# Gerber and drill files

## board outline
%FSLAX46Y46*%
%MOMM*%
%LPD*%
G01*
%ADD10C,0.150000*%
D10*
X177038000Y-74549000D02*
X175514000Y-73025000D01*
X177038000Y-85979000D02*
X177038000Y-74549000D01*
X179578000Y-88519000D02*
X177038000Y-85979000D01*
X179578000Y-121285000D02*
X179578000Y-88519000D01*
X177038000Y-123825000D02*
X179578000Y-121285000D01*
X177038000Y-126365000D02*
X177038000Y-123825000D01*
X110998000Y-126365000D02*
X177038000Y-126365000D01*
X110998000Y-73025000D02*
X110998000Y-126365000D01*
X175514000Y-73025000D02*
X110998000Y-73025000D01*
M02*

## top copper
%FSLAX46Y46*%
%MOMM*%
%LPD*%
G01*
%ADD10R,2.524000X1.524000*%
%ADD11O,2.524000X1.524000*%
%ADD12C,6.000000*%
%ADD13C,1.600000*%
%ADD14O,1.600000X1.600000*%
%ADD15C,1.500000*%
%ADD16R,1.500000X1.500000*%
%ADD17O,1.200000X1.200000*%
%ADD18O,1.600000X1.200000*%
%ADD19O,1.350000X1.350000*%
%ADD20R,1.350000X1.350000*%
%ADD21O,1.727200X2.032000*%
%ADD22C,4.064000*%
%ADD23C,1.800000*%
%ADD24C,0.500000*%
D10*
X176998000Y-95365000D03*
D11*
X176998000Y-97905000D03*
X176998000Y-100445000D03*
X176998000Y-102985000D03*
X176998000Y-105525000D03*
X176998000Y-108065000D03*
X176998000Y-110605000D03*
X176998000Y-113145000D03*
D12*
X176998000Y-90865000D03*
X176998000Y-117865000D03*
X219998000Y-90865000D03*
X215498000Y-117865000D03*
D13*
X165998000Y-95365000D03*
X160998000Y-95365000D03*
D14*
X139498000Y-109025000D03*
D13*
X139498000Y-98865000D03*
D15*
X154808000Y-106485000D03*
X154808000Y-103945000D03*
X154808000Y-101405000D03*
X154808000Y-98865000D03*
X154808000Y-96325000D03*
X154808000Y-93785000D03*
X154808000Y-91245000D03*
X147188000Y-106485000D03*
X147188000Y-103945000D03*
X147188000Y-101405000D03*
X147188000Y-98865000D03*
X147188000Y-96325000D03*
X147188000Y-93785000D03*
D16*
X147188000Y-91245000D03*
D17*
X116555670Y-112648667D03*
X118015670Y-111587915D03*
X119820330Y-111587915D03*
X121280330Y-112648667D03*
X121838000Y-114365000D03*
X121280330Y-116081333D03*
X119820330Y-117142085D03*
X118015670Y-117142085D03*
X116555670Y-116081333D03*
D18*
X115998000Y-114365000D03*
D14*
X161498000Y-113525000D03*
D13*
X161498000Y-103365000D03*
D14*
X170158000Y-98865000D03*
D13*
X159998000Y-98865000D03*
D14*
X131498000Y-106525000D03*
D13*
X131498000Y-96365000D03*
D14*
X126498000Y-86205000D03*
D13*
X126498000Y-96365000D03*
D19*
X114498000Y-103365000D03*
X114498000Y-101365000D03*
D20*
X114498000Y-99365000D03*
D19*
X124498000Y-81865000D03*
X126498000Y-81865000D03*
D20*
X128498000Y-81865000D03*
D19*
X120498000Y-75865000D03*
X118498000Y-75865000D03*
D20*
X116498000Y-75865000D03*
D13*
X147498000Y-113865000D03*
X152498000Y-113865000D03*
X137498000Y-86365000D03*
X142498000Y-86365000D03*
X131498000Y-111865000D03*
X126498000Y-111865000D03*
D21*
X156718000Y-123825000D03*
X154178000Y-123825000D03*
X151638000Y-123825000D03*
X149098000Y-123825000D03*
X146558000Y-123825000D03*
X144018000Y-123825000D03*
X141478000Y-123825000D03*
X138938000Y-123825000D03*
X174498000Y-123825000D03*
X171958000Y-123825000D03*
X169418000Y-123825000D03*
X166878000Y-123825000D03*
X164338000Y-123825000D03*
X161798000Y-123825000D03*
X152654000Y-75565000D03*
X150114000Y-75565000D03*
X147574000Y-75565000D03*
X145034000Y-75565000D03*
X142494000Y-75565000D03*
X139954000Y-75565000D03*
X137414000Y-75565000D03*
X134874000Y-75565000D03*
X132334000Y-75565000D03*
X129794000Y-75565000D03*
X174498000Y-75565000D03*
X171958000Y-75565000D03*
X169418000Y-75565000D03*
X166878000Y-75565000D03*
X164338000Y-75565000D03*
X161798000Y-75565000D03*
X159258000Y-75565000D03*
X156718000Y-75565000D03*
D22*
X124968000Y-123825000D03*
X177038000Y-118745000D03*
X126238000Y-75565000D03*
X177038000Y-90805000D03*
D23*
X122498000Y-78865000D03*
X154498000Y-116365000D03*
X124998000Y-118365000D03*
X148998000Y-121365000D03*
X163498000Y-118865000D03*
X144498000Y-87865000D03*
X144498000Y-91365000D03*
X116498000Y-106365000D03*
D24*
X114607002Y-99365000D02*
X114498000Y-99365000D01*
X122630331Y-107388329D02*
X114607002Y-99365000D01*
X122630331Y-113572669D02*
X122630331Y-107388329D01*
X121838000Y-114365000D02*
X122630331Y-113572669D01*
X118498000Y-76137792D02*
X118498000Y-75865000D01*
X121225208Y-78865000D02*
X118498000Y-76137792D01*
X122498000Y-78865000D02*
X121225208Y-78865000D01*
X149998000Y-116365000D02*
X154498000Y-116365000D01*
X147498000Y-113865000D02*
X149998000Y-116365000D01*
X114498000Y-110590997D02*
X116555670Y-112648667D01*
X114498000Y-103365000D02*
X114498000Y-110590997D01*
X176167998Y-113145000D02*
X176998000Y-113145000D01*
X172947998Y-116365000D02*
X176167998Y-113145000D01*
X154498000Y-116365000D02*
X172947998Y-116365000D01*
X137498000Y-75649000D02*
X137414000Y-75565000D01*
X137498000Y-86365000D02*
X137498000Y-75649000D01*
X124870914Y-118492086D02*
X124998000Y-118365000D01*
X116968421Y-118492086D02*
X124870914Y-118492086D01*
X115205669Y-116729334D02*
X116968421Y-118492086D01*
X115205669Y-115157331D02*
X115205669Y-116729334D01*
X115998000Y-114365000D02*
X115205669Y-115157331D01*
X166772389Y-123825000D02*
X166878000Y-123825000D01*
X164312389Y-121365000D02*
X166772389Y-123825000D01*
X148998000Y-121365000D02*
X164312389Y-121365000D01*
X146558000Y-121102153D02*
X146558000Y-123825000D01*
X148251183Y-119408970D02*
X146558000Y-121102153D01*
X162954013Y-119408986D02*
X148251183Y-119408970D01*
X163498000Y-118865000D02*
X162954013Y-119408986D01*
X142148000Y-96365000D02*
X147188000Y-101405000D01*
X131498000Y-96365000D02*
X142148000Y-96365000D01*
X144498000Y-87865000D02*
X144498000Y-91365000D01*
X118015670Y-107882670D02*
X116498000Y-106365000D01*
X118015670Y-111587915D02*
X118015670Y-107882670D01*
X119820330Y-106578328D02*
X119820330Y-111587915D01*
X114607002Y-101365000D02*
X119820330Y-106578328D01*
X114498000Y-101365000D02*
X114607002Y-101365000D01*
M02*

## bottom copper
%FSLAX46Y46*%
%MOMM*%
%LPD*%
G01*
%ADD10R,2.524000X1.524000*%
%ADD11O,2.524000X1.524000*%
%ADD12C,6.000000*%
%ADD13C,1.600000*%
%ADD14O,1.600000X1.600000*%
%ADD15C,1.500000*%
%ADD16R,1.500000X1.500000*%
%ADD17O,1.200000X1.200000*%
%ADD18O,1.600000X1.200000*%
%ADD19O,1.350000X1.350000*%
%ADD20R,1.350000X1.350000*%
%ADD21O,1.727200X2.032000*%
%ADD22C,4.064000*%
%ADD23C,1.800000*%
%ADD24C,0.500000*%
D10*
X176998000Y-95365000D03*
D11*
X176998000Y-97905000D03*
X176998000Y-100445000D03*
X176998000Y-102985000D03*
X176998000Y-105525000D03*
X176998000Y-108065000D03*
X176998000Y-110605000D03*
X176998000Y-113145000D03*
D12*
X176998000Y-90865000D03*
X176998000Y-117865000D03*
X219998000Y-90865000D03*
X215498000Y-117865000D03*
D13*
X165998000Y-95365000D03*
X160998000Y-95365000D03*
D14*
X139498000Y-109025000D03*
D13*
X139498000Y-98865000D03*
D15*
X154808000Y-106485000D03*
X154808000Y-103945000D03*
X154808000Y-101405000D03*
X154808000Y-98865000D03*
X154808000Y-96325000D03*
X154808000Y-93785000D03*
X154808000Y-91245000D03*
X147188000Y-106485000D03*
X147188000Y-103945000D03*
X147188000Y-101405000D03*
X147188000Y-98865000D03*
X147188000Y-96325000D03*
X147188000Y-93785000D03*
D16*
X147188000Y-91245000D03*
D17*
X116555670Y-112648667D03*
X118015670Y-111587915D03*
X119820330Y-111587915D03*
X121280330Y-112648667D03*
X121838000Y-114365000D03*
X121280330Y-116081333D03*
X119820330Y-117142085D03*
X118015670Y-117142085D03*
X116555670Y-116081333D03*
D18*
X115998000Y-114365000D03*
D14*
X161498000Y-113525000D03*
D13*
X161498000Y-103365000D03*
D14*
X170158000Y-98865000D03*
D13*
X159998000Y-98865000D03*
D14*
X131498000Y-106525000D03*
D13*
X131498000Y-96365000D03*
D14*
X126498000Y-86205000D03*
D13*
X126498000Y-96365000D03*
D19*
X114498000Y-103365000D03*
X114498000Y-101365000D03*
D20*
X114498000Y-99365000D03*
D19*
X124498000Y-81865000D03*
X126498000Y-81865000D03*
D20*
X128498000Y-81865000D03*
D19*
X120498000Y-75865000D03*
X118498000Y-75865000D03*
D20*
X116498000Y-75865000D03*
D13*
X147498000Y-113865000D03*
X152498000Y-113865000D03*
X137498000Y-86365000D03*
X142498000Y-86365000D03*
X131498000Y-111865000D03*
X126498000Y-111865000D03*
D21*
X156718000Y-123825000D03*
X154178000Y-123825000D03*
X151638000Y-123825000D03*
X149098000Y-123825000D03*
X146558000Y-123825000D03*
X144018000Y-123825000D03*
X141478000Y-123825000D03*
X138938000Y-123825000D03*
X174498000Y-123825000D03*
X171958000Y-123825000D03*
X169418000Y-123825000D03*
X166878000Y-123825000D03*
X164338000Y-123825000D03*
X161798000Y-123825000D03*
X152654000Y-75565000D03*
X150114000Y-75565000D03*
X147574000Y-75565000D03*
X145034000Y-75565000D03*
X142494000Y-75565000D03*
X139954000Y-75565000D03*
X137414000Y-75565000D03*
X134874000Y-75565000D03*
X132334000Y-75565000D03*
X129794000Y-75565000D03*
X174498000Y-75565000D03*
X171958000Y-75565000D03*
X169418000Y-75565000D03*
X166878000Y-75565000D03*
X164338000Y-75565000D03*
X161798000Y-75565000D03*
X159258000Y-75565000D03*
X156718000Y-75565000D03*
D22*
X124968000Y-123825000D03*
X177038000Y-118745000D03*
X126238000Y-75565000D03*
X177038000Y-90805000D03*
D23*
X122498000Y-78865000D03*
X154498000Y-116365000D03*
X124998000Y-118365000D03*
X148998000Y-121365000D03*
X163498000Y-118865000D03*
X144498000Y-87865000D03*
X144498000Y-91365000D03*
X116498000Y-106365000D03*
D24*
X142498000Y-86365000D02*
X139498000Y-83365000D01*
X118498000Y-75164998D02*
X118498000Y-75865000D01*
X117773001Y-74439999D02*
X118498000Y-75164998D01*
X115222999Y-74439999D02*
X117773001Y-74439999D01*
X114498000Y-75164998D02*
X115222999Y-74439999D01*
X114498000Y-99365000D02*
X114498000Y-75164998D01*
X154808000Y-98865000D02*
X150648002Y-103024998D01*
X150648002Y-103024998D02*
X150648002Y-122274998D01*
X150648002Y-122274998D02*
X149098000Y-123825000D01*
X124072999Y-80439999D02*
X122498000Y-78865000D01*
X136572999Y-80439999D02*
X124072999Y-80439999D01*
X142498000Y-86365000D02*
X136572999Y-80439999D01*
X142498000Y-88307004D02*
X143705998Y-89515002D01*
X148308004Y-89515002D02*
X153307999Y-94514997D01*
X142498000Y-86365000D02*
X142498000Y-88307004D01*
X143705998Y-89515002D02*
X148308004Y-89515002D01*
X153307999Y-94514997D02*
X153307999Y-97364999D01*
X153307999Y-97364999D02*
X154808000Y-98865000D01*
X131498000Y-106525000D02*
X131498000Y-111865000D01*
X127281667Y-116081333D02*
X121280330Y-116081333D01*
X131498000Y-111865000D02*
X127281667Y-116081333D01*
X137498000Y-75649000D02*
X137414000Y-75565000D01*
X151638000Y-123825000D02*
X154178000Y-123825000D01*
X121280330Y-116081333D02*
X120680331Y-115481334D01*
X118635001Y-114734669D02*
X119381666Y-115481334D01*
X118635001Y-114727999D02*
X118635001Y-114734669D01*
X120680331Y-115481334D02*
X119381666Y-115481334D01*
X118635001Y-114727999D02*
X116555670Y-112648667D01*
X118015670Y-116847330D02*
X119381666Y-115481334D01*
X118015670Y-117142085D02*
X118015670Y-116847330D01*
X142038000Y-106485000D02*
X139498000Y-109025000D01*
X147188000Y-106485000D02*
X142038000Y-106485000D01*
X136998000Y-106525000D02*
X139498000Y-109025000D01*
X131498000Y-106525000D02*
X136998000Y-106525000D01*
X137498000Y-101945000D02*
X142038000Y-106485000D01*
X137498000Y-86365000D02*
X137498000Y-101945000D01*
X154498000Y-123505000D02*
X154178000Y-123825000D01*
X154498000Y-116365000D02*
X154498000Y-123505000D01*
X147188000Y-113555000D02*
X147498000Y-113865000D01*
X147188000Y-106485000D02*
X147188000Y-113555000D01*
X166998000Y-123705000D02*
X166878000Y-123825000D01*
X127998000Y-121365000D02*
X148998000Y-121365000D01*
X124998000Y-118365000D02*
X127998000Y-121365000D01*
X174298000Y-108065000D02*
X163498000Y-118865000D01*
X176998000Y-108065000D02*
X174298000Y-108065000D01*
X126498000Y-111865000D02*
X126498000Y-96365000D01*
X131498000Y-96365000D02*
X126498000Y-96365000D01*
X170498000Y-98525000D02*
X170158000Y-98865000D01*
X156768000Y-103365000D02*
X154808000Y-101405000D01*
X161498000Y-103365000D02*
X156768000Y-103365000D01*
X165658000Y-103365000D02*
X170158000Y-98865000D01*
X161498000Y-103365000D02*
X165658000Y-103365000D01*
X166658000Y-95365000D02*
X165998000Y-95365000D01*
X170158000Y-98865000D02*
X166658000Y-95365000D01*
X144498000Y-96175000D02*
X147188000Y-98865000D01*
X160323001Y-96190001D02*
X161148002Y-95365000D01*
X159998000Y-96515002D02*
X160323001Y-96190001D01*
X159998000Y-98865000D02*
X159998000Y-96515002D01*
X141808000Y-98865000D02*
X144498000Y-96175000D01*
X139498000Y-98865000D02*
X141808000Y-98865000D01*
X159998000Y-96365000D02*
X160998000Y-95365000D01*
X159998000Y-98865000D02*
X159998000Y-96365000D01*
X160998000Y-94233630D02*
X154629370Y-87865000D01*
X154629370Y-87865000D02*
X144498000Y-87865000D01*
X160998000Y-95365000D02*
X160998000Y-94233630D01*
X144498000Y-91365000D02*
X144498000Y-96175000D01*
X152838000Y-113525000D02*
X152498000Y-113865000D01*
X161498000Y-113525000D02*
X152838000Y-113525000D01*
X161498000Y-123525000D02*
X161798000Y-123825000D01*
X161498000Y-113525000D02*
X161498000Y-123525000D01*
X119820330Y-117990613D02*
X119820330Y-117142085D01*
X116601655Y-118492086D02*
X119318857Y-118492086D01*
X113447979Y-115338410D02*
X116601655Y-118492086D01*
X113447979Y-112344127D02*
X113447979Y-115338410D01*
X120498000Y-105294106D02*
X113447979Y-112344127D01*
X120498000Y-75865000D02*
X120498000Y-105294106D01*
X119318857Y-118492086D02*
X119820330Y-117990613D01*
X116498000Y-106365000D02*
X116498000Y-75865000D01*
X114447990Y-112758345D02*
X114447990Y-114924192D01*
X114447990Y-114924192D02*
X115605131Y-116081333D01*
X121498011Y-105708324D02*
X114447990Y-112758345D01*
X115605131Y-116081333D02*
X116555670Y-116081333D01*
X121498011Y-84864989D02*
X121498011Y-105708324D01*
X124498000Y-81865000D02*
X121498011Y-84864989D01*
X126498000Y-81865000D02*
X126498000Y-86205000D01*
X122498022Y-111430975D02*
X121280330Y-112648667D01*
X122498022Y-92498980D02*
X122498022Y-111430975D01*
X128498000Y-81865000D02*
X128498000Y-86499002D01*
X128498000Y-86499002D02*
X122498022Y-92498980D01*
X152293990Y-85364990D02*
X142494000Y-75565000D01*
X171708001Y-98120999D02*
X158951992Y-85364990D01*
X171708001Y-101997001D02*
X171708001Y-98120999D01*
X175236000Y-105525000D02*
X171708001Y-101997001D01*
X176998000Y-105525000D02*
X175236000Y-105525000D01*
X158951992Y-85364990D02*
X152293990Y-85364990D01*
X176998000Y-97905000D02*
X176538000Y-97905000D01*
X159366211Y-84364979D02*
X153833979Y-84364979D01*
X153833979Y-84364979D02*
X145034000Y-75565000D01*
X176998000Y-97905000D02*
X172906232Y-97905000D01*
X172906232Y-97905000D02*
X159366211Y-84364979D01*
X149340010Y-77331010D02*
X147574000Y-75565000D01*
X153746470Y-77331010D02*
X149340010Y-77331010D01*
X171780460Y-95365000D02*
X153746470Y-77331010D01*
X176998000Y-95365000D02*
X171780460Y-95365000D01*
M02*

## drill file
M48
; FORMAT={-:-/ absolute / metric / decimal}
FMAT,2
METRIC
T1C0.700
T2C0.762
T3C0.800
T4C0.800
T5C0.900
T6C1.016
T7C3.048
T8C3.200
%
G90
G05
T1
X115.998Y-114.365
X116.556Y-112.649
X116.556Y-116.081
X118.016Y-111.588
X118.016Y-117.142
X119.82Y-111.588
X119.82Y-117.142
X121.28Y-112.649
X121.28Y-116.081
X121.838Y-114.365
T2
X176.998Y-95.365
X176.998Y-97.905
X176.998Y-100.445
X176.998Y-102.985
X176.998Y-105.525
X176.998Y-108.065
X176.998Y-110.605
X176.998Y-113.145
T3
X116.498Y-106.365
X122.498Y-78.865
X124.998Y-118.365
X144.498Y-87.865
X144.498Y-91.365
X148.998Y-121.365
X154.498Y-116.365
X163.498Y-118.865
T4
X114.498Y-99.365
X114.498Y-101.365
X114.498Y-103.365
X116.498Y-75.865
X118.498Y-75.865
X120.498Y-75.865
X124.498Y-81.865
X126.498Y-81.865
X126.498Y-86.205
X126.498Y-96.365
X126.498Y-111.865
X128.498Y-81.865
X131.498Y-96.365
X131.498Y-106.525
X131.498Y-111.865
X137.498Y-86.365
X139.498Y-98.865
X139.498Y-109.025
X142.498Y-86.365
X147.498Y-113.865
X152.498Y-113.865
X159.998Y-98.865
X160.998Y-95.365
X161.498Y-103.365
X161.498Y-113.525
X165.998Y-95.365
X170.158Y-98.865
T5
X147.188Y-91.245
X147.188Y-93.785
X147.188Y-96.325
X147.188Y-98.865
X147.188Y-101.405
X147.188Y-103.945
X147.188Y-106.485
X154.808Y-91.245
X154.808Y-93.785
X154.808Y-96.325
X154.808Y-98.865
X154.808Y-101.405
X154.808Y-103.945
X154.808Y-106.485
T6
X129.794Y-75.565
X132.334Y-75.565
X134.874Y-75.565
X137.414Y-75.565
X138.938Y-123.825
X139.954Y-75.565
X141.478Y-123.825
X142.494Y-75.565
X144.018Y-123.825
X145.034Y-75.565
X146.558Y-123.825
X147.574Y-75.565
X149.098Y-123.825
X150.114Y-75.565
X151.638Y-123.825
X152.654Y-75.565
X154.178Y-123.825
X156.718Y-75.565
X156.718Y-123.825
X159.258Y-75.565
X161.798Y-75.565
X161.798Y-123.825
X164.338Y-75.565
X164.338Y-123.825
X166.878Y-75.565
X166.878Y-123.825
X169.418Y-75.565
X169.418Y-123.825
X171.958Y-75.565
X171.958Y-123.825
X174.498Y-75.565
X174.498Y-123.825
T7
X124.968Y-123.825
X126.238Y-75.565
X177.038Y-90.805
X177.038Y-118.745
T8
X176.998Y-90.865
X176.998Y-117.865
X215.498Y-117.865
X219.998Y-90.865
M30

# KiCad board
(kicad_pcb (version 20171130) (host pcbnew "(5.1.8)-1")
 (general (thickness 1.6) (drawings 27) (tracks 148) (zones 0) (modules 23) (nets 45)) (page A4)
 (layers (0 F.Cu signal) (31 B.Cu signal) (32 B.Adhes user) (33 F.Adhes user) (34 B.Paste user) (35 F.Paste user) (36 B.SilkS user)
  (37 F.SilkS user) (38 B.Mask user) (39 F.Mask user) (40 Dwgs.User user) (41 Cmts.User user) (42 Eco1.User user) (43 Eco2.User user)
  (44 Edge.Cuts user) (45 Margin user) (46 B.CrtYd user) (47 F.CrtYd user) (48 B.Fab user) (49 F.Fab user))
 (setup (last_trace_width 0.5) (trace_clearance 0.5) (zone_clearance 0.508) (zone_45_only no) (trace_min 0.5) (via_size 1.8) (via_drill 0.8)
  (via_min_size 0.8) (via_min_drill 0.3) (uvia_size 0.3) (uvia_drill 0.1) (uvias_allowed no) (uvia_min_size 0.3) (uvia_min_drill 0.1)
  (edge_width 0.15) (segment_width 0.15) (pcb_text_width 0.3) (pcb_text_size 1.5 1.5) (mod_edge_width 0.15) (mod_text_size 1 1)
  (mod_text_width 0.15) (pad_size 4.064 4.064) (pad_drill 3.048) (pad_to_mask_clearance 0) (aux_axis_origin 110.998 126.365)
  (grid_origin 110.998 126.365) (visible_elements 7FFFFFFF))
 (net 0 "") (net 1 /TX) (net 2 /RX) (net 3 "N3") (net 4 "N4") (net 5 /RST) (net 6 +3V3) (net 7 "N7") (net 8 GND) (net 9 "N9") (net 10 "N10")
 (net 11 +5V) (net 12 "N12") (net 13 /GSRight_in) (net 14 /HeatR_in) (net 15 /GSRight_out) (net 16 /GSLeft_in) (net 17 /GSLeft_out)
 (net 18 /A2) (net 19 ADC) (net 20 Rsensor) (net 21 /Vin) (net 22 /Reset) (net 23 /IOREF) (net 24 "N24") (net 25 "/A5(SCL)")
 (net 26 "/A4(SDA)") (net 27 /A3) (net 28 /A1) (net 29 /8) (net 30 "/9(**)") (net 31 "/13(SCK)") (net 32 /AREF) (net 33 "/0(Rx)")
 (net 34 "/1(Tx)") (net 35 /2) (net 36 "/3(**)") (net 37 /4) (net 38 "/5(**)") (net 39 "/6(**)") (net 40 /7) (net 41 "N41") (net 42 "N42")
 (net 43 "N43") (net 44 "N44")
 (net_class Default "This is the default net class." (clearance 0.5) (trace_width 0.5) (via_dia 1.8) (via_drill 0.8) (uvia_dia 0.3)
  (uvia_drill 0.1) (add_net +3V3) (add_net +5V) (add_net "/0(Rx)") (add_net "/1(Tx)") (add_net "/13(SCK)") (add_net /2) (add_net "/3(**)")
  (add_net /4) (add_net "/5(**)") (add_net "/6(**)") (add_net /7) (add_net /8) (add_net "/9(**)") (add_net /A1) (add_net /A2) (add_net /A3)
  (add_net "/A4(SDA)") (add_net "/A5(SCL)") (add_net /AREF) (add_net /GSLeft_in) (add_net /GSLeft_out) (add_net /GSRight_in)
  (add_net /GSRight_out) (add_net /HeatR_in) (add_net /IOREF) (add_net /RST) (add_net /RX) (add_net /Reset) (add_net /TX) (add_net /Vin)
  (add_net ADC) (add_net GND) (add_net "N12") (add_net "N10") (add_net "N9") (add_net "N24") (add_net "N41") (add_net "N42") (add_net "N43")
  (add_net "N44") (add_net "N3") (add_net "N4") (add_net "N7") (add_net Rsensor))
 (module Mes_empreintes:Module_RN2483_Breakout (layer F.Cu) (at 176.998 95.365 270)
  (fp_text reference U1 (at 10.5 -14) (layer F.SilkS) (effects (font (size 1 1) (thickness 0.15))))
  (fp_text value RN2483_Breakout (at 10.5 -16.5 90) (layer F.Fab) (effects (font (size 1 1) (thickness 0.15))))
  (pad 1 thru_hole rect (at 0 0 270) (size 1.524 2.524) (drill 0.762) (layers *.Cu *.Mask) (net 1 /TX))
  (pad 2 thru_hole oval (at 2.54 0 270) (size 1.524 2.524) (drill 0.762) (layers *.Cu *.Mask) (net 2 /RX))
  (pad 3 thru_hole oval (at 5.08 0 270) (size 1.524 2.524) (drill 0.762) (layers *.Cu *.Mask) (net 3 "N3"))
  (pad 4 thru_hole oval (at 7.62 0 270) (size 1.524 2.524) (drill 0.762) (layers *.Cu *.Mask) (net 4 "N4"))
  (pad 5 thru_hole oval (at 10.16 0 270) (size 1.524 2.524) (drill 0.762) (layers *.Cu *.Mask) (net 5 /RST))
  (pad 6 thru_hole oval (at 12.7 0 270) (size 1.524 2.524) (drill 0.762) (layers *.Cu *.Mask) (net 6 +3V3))
  (pad 7 thru_hole oval (at 15.24 0 270) (size 1.524 2.524) (drill 0.762) (layers *.Cu *.Mask) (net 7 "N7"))
  (pad 8 thru_hole oval (at 17.78 0 270) (size 1.524 2.524) (drill 0.762) (layers *.Cu *.Mask) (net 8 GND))
  (pad "" np_thru_hole circle (at -4.5 0 270) (size 6 6) (drill 3.2) (layers *.Cu *.Mask))
  (pad "" np_thru_hole circle (at 22.5 0 270) (size 6 6) (drill 3.2) (layers *.Cu *.Mask))
  (pad "" np_thru_hole circle (at -4.5 -43 270) (size 6 6) (drill 3.2) (layers *.Cu *.Mask))
  (pad "" np_thru_hole circle (at 22.5 -38.5 270) (size 6 6) (drill 3.2) (layers *.Cu *.Mask)))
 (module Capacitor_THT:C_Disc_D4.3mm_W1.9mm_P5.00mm (layer F.Cu) (at 160.998 95.365)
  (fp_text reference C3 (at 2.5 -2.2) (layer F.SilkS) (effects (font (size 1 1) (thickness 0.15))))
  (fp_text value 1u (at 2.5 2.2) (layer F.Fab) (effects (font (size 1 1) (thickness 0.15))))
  (pad 2 thru_hole circle (at 5 0) (size 1.6 1.6) (drill 0.8) (layers *.Cu *.Mask) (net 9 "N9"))
  (pad 1 thru_hole circle (at 0 0) (size 1.6 1.6) (drill 0.8) (layers *.Cu *.Mask) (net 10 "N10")))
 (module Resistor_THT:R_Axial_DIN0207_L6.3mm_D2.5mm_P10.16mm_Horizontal (layer F.Cu) (at 139.498 98.865 270)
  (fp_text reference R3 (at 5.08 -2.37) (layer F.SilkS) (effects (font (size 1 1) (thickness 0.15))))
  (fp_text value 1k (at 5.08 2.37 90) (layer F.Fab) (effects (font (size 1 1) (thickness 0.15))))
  (pad 2 thru_hole oval (at 10.16 0 270) (size 1.6 1.6) (drill 0.8) (layers *.Cu *.Mask) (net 8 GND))
  (pad 1 thru_hole circle (at 0 0 270) (size 1.6 1.6) (drill 0.8) (layers *.Cu *.Mask) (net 10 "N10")))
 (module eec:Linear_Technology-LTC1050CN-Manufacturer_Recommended (layer F.Cu) (at 150.998 98.865)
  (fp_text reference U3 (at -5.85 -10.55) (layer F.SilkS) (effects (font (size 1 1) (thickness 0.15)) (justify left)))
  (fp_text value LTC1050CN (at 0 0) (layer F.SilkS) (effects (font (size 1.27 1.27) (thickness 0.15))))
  (pad 8 thru_hole circle (at 3.81 7.62) (size 1.5 1.5) (drill 0.900001) (layers *.Cu))
  (pad 9 thru_hole circle (at 3.81 5.08) (size 1.5 1.5) (drill 0.900001) (layers *.Cu))
  (pad 10 thru_hole circle (at 3.81 2.54) (size 1.5 1.5) (drill 0.900001) (layers *.Cu) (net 9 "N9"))
  (pad 11 thru_hole circle (at 3.81 0) (size 1.5 1.5) (drill 0.900001) (layers *.Cu) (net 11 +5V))
  (pad 12 thru_hole circle (at 3.81 -2.54) (size 1.5 1.5) (drill 0.900001) (layers *.Cu))
  (pad 13 thru_hole circle (at 3.81 -5.08) (size 1.5 1.5) (drill 0.900001) (layers *.Cu))
  (pad 14 thru_hole circle (at 3.81 -7.62) (size 1.5 1.5) (drill 0.900001) (layers *.Cu))
  (pad 7 thru_hole circle (at -3.81 7.62) (size 1.5 1.5) (drill 0.900001) (layers *.Cu) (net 8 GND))
  (pad 6 thru_hole circle (at -3.81 5.08) (size 1.5 1.5) (drill 0.900001) (layers *.Cu))
  (pad 5 thru_hole circle (at -3.81 2.54) (size 1.5 1.5) (drill 0.900001) (layers *.Cu) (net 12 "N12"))
  (pad 4 thru_hole circle (at -3.81 0) (size 1.5 1.5) (drill 0.900001) (layers *.Cu) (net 10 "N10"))
  (pad 3 thru_hole circle (at -3.81 -2.54) (size 1.5 1.5) (drill 0.900001) (layers *.Cu))
  (pad 2 thru_hole circle (at -3.81 -5.08) (size 1.5 1.5) (drill 0.900001) (layers *.Cu))
  (pad 1 thru_hole rect (at -3.81 -7.62) (size 1.5 1.5) (drill 0.900001) (layers *.Cu)))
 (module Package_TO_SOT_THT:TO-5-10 (layer F.Cu) (at 115.998 114.365)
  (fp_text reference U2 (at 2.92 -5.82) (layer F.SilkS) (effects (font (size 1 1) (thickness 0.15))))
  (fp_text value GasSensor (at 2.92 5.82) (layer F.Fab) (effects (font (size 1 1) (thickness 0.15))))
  (pad 10 thru_hole oval (at 0.55767 -1.716333) (size 1.2 1.2) (drill 0.7) (layers *.Cu *.Mask) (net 8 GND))
  (pad 9 thru_hole oval (at 2.01767 -2.777085) (size 1.2 1.2) (drill 0.7) (layers *.Cu *.Mask) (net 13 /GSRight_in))
  (pad 8 thru_hole oval (at 3.82233 -2.777085) (size 1.2 1.2) (drill 0.7) (layers *.Cu *.Mask) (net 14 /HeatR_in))
  (pad 7 thru_hole oval (at 5.28233 -1.716333) (size 1.2 1.2) (drill 0.7) (layers *.Cu *.Mask) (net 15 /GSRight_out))
  (pad 6 thru_hole oval (at 5.84 0) (size 1.2 1.2) (drill 0.7) (layers *.Cu *.Mask) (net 11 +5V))
  (pad 5 thru_hole oval (at 5.28233 1.716333) (size 1.2 1.2) (drill 0.7) (layers *.Cu *.Mask) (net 8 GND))
  (pad 4 thru_hole oval (at 3.82233 2.777085) (size 1.2 1.2) (drill 0.7) (layers *.Cu *.Mask) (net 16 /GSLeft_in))
  (pad 3 thru_hole oval (at 2.01767 2.777085) (size 1.2 1.2) (drill 0.7) (layers *.Cu *.Mask) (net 8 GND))
  (pad 2 thru_hole oval (at 0.55767 1.716333) (size 1.2 1.2) (drill 0.7) (layers *.Cu *.Mask) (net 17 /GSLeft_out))
  (pad 1 thru_hole oval (at 0 0) (size 1.6 1.2) (drill 0.7) (layers *.Cu *.Mask) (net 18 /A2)))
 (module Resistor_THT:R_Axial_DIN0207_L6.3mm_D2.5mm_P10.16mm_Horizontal (layer F.Cu) (at 161.498 103.365 270)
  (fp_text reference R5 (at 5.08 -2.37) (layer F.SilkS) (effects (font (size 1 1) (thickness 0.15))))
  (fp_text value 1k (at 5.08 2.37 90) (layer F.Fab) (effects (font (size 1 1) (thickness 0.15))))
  (pad 2 thru_hole oval (at 10.16 0 270) (size 1.6 1.6) (drill 0.8) (layers *.Cu *.Mask) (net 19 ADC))
  (pad 1 thru_hole circle (at 0 0 270) (size 1.6 1.6) (drill 0.8) (layers *.Cu *.Mask) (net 9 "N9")))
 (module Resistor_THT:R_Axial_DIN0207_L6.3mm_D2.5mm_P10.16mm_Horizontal (layer F.Cu) (at 159.998 98.865)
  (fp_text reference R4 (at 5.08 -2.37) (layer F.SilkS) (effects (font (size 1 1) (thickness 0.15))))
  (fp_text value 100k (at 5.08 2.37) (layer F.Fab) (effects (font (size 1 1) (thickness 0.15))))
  (pad 2 thru_hole oval (at 10.16 0) (size 1.6 1.6) (drill 0.8) (layers *.Cu *.Mask) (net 9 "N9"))
  (pad 1 thru_hole circle (at 0 0) (size 1.6 1.6) (drill 0.8) (layers *.Cu *.Mask) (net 10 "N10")))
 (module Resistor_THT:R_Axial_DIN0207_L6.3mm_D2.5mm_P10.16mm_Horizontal (layer F.Cu) (at 131.498 96.365 270)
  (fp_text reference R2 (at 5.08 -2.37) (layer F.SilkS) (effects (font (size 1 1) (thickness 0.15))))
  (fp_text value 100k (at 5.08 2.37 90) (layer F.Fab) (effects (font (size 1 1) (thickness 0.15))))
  (pad 2 thru_hole oval (at 10.16 0 270) (size 1.6 1.6) (drill 0.8) (layers *.Cu *.Mask) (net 8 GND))
  (pad 1 thru_hole circle (at 0 0 270) (size 1.6 1.6) (drill 0.8) (layers *.Cu *.Mask) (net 12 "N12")))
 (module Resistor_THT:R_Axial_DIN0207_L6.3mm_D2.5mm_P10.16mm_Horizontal (layer F.Cu) (at 126.498 96.365 90)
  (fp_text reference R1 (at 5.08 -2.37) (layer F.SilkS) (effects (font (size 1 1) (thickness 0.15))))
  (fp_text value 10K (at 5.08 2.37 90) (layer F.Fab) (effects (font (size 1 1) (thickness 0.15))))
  (pad 2 thru_hole oval (at 10.16 0 90) (size 1.6 1.6) (drill 0.8) (layers *.Cu *.Mask) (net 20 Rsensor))
  (pad 1 thru_hole circle (at 0 0 90) (size 1.6 1.6) (drill 0.8) (layers *.Cu *.Mask) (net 12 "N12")))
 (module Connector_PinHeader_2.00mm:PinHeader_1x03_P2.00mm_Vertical (layer F.Cu) (at 114.498 99.365)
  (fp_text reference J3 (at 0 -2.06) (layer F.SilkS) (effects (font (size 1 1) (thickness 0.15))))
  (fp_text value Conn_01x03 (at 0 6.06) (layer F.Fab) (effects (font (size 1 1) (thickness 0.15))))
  (pad 3 thru_hole oval (at 0 4) (size 1.35 1.35) (drill 0.8) (layers *.Cu *.Mask) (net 8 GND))
  (pad 2 thru_hole oval (at 0 2) (size 1.35 1.35) (drill 0.8) (layers *.Cu *.Mask) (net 14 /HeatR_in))
  (pad 1 thru_hole rect (at 0 0) (size 1.35 1.35) (drill 0.8) (layers *.Cu *.Mask) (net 11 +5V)))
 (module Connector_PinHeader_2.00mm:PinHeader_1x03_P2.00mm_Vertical (layer F.Cu) (at 128.498 81.865 270)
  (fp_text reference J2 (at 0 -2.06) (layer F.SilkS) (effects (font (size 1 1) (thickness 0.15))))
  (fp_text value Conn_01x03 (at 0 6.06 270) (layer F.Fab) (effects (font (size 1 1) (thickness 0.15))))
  (pad 3 thru_hole oval (at 0 4 270) (size 1.35 1.35) (drill 0.8) (layers *.Cu *.Mask) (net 17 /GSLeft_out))
  (pad 2 thru_hole oval (at 0 2 270) (size 1.35 1.35) (drill 0.8) (layers *.Cu *.Mask) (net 20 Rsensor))
  (pad 1 thru_hole rect (at 0 0 270) (size 1.35 1.35) (drill 0.8) (layers *.Cu *.Mask) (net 15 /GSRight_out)))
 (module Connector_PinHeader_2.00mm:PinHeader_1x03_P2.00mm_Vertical (layer F.Cu) (at 116.498 75.865 90)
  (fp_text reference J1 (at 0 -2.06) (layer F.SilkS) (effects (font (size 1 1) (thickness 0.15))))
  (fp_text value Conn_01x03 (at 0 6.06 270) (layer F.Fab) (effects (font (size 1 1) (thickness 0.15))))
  (pad 3 thru_hole oval (at 0 4 90) (size 1.35 1.35) (drill 0.8) (layers *.Cu *.Mask) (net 16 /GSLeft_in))
  (pad 2 thru_hole oval (at 0 2 90) (size 1.35 1.35) (drill 0.8) (layers *.Cu *.Mask) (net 11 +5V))
  (pad 1 thru_hole rect (at 0 0 90) (size 1.35 1.35) (drill 0.8) (layers *.Cu *.Mask) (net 13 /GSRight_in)))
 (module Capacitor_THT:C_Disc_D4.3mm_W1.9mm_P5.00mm (layer F.Cu) (at 152.498 113.865 180)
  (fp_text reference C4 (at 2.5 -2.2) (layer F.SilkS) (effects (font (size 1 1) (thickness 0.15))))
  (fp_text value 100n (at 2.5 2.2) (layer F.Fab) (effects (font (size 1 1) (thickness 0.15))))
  (pad 2 thru_hole circle (at 5 0 180) (size 1.6 1.6) (drill 0.8) (layers *.Cu *.Mask) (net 8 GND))
  (pad 1 thru_hole circle (at 0 0 180) (size 1.6 1.6) (drill 0.8) (layers *.Cu *.Mask) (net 19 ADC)))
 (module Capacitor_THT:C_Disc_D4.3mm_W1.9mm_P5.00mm (layer F.Cu) (at 142.498 86.365 180)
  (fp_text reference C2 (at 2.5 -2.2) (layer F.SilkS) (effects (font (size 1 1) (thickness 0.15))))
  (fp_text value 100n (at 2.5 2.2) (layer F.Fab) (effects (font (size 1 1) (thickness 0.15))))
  (pad 2 thru_hole circle (at 5 0 180) (size 1.6 1.6) (drill 0.8) (layers *.Cu *.Mask) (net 8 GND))
  (pad 1 thru_hole circle (at 0 0 180) (size 1.6 1.6) (drill 0.8) (layers *.Cu *.Mask) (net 11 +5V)))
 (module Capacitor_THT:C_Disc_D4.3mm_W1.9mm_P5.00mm (layer F.Cu) (at 126.498 111.865)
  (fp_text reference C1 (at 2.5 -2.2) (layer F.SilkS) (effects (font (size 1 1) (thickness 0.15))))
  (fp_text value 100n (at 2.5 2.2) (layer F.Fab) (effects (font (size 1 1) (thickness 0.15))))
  (pad 2 thru_hole circle (at 5 0) (size 1.6 1.6) (drill 0.8) (layers *.Cu *.Mask) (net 8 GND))
  (pad 1 thru_hole circle (at 0 0) (size 1.6 1.6) (drill 0.8) (layers *.Cu *.Mask) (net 12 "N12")))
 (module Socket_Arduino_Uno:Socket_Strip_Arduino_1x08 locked (layer F.Cu) (at 138.938 123.825)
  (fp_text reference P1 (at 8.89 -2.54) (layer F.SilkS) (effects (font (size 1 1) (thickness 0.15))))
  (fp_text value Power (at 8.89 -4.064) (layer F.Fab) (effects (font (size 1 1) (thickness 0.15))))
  (pad 8 thru_hole oval (at 17.78 0) (size 1.7272 2.032) (drill 1.016) (layers *.Cu *.Mask F.SilkS) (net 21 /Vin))
  (pad 7 thru_hole oval (at 15.24 0) (size 1.7272 2.032) (drill 1.016) (layers *.Cu *.Mask F.SilkS) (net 8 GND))
  (pad 6 thru_hole oval (at 12.7 0) (size 1.7272 2.032) (drill 1.016) (layers *.Cu *.Mask F.SilkS) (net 8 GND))
  (pad 5 thru_hole oval (at 10.16 0) (size 1.7272 2.032) (drill 1.016) (layers *.Cu *.Mask F.SilkS) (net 11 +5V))
  (pad 4 thru_hole oval (at 7.62 0) (size 1.7272 2.032) (drill 1.016) (layers *.Cu *.Mask F.SilkS) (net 6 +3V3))
  (pad 3 thru_hole oval (at 5.08 0) (size 1.7272 2.032) (drill 1.016) (layers *.Cu *.Mask F.SilkS) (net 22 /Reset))
  (pad 2 thru_hole oval (at 2.54 0) (size 1.7272 2.032) (drill 1.016) (layers *.Cu *.Mask F.SilkS) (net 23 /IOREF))
  (pad 1 thru_hole oval (at 0 0) (size 1.7272 2.032) (drill 1.016) (layers *.Cu *.Mask F.SilkS) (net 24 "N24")))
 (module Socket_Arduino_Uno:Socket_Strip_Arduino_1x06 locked (layer F.Cu) (at 161.798 123.825)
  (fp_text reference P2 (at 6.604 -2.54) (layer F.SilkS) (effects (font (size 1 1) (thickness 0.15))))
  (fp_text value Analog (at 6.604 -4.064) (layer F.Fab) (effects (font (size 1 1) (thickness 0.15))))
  (pad 6 thru_hole oval (at 12.7 0) (size 1.7272 2.032) (drill 1.016) (layers *.Cu *.Mask F.SilkS) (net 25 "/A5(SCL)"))
  (pad 5 thru_hole oval (at 10.16 0) (size 1.7272 2.032) (drill 1.016) (layers *.Cu *.Mask F.SilkS) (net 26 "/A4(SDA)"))
  (pad 4 thru_hole oval (at 7.62 0) (size 1.7272 2.032) (drill 1.016) (layers *.Cu *.Mask F.SilkS) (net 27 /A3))
  (pad 3 thru_hole oval (at 5.08 0) (size 1.7272 2.032) (drill 1.016) (layers *.Cu *.Mask F.SilkS) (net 18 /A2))
  (pad 2 thru_hole oval (at 2.54 0) (size 1.7272 2.032) (drill 1.016) (layers *.Cu *.Mask F.SilkS) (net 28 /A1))
  (pad 1 thru_hole oval (at 0 0) (size 1.7272 2.032) (drill 1.016) (layers *.Cu *.Mask F.SilkS) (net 19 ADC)))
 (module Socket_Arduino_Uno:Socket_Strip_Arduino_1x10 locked (layer F.Cu) (at 129.794 75.565)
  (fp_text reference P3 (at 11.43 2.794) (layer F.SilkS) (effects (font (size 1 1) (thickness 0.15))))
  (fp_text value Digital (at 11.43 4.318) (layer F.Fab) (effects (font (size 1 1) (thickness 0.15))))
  (pad 10 thru_hole oval (at 22.86 0) (size 1.7272 2.032) (drill 1.016) (layers *.Cu *.Mask F.SilkS) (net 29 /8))
  (pad 9 thru_hole oval (at 20.32 0) (size 1.7272 2.032) (drill 1.016) (layers *.Cu *.Mask F.SilkS) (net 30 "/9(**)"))
  (pad 8 thru_hole oval (at 17.78 0) (size 1.7272 2.032) (drill 1.016) (layers *.Cu *.Mask F.SilkS) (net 1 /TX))
  (pad 7 thru_hole oval (at 15.24 0) (size 1.7272 2.032) (drill 1.016) (layers *.Cu *.Mask F.SilkS) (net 2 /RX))
  (pad 6 thru_hole oval (at 12.7 0) (size 1.7272 2.032) (drill 1.016) (layers *.Cu *.Mask F.SilkS) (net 5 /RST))
  (pad 5 thru_hole oval (at 10.16 0) (size 1.7272 2.032) (drill 1.016) (layers *.Cu *.Mask F.SilkS) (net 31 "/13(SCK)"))
  (pad 4 thru_hole oval (at 7.62 0) (size 1.7272 2.032) (drill 1.016) (layers *.Cu *.Mask F.SilkS) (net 8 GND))
  (pad 3 thru_hole oval (at 5.08 0) (size 1.7272 2.032) (drill 1.016) (layers *.Cu *.Mask F.SilkS) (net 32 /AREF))
  (pad 2 thru_hole oval (at 2.54 0) (size 1.7272 2.032) (drill 1.016) (layers *.Cu *.Mask F.SilkS) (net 26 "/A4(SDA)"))
  (pad 1 thru_hole oval (at 0 0) (size 1.7272 2.032) (drill 1.016) (layers *.Cu *.Mask F.SilkS) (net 25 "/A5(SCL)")))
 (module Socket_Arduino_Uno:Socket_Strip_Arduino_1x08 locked (layer F.Cu) (at 156.718 75.565)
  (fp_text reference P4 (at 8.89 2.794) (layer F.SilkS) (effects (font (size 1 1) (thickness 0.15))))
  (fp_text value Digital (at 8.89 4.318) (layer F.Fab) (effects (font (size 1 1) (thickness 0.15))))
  (pad 8 thru_hole oval (at 17.78 0) (size 1.7272 2.032) (drill 1.016) (layers *.Cu *.Mask F.SilkS) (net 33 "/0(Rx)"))
  (pad 7 thru_hole oval (at 15.24 0) (size 1.7272 2.032) (drill 1.016) (layers *.Cu *.Mask F.SilkS) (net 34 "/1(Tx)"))
  (pad 6 thru_hole oval (at 12.7 0) (size 1.7272 2.032) (drill 1.016) (layers *.Cu *.Mask F.SilkS) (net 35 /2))
  (pad 5 thru_hole oval (at 10.16 0) (size 1.7272 2.032) (drill 1.016) (layers *.Cu *.Mask F.SilkS) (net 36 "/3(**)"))
  (pad 4 thru_hole oval (at 7.62 0) (size 1.7272 2.032) (drill 1.016) (layers *.Cu *.Mask F.SilkS) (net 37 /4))
  (pad 3 thru_hole oval (at 5.08 0) (size 1.7272 2.032) (drill 1.016) (layers *.Cu *.Mask F.SilkS) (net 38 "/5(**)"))
  (pad 2 thru_hole oval (at 2.54 0) (size 1.7272 2.032) (drill 1.016) (layers *.Cu *.Mask F.SilkS) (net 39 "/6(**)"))
  (pad 1 thru_hole oval (at 0 0) (size 1.7272 2.032) (drill 1.016) (layers *.Cu *.Mask F.SilkS) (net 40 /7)))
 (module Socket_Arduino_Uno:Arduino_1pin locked (layer F.Cu) (at 124.968 123.825)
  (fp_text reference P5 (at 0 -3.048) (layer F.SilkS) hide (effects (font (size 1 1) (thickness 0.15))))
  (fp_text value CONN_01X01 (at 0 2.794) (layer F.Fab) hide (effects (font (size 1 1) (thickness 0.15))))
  (pad 1 thru_hole circle (at 0 0) (size 4.064 4.064) (drill 3.048) (layers *.Cu *.Mask F.SilkS) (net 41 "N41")))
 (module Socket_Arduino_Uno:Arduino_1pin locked (layer F.Cu) (at 177.038 118.745)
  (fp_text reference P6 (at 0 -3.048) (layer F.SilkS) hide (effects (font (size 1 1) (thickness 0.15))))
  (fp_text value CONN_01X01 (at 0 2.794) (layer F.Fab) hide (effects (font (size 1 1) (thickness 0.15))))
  (pad 1 thru_hole circle (at 0 0) (size 4.064 4.064) (drill 3.048) (layers *.Cu *.Mask F.SilkS) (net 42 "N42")))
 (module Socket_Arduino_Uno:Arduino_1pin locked (layer F.Cu) (at 126.238 75.565)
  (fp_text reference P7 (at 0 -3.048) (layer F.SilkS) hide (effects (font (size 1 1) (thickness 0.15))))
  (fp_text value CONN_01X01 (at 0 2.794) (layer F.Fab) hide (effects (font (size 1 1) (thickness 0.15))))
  (pad 1 thru_hole circle (at 0 0) (size 4.064 4.064) (drill 3.048) (layers *.Cu *.Mask F.SilkS) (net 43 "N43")))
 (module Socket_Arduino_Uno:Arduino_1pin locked (layer F.Cu) (at 177.038 90.805)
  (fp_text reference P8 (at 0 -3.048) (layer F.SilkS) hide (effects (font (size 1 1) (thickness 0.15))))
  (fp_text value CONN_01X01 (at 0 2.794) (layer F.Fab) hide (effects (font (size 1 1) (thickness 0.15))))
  (pad 1 thru_hole circle (at 0 0) (size 4.064 4.064) (drill 3.048) (layers *.Cu *.Mask F.SilkS) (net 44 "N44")))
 (gr_line (start 177.038 74.549) (end 175.514 73.025) (angle 90) (layer Edge.Cuts) (width 0.15))
 (gr_line (start 177.038 85.979) (end 177.038 74.549) (angle 90) (layer Edge.Cuts) (width 0.15))
 (gr_line (start 179.578 88.519) (end 177.038 85.979) (angle 90) (layer Edge.Cuts) (width 0.15))
 (gr_line (start 179.578 121.285) (end 179.578 88.519) (angle 90) (layer Edge.Cuts) (width 0.15))
 (gr_line (start 177.038 123.825) (end 179.578 121.285) (angle 90) (layer Edge.Cuts) (width 0.15))
 (gr_line (start 177.038 126.365) (end 177.038 123.825) (angle 90) (layer Edge.Cuts) (width 0.15))
 (gr_line (start 110.998 126.365) (end 177.038 126.365) (angle 90) (layer Edge.Cuts) (width 0.15))
 (gr_line (start 110.998 73.025) (end 110.998 126.365) (angle 90) (layer Edge.Cuts) (width 0.15))
 (gr_line (start 175.514 73.025) (end 110.998 73.025) (angle 90) (layer Edge.Cuts) (width 0.15))
 (segment (start 114.607002 99.365) (end 114.498 99.365) (width 0.5) (layer F.Cu) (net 11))
 (segment (start 122.630331 107.388329) (end 114.607002 99.365) (width 0.5) (layer F.Cu) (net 11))
 (segment (start 122.630331 113.572669) (end 122.630331 107.388329) (width 0.5) (layer F.Cu) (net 11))
 (segment (start 121.838 114.365) (end 122.630331 113.572669) (width 0.5) (layer F.Cu) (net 11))
 (segment (start 142.498 86.365) (end 139.498 83.365) (width 0.5) (layer B.Cu) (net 11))
 (via (at 122.498 78.865) (size 1.8) (drill 0.8) (layers F.Cu B.Cu) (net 11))
 (segment (start 118.498 76.137792) (end 118.498 75.865) (width 0.5) (layer F.Cu) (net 11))
 (segment (start 121.225208 78.865) (end 118.498 76.137792) (width 0.5) (layer F.Cu) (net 11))
 (segment (start 122.498 78.865) (end 121.225208 78.865) (width 0.5) (layer F.Cu) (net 11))
 (segment (start 118.498 75.164998) (end 118.498 75.865) (width 0.5) (layer B.Cu) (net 11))
 (segment (start 117.773001 74.439999) (end 118.498 75.164998) (width 0.5) (layer B.Cu) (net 11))
 (segment (start 115.222999 74.439999) (end 117.773001 74.439999) (width 0.5) (layer B.Cu) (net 11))
 (segment (start 114.498 75.164998) (end 115.222999 74.439999) (width 0.5) (layer B.Cu) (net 11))
 (segment (start 114.498 99.365) (end 114.498 75.164998) (width 0.5) (layer B.Cu) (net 11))
 (segment (start 154.808 98.865) (end 150.648002 103.024998) (width 0.5) (layer B.Cu) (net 11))
 (segment (start 150.648002 103.024998) (end 150.648002 122.274998) (width 0.5) (layer B.Cu) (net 11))
 (segment (start 150.648002 122.274998) (end 149.098 123.825) (width 0.5) (layer B.Cu) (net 11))
 (segment (start 124.072999 80.439999) (end 122.498 78.865) (width 0.5) (layer B.Cu) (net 11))
 (segment (start 136.572999 80.439999) (end 124.072999 80.439999) (width 0.5) (layer B.Cu) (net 11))
 (segment (start 142.498 86.365) (end 136.572999 80.439999) (width 0.5) (layer B.Cu) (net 11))
 (segment (start 142.498 88.307004) (end 143.705998 89.515002) (width 0.5) (layer B.Cu) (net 11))
 (segment (start 148.308004 89.515002) (end 153.307999 94.514997) (width 0.5) (layer B.Cu) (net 11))
 (segment (start 142.498 86.365) (end 142.498 88.307004) (width 0.5) (layer B.Cu) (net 11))
 (segment (start 143.705998 89.515002) (end 148.308004 89.515002) (width 0.5) (layer B.Cu) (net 11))
 (segment (start 153.307999 94.514997) (end 153.307999 97.364999) (width 0.5) (layer B.Cu) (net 11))
 (segment (start 153.307999 97.364999) (end 154.808 98.865) (width 0.5) (layer B.Cu) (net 11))
 (segment (start 131.498 106.525) (end 131.498 111.865) (width 0.5) (layer B.Cu) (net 8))
 (segment (start 127.281667 116.081333) (end 121.28033 116.081333) (width 0.5) (layer B.Cu) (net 8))
 (segment (start 131.498 111.865) (end 127.281667 116.081333) (width 0.5) (layer B.Cu) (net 8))
 (segment (start 137.498 75.649) (end 137.414 75.565) (width 0.5) (layer B.Cu) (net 8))
 (segment (start 151.638 123.825) (end 154.178 123.825) (width 0.5) (layer B.Cu) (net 8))
 (segment (start 121.28033 116.081333) (end 120.680331 115.481334) (width 0.5) (layer B.Cu) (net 8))
 (segment (start 118.635001 114.734669) (end 119.381666 115.481334) (width 0.5) (layer B.Cu) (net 8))
 (segment (start 118.635001 114.727999) (end 118.635001 114.734669) (width 0.5) (layer B.Cu) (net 8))
 (segment (start 120.680331 115.481334) (end 119.381666 115.481334) (width 0.5) (layer B.Cu) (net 8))
 (segment (start 118.635001 114.727999) (end 116.55567 112.648667) (width 0.5) (layer B.Cu) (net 8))
 (segment (start 118.01567 116.84733) (end 119.381666 115.481334) (width 0.5) (layer B.Cu) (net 8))
 (segment (start 118.01567 117.142085) (end 118.01567 116.84733) (width 0.5) (layer B.Cu) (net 8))
 (segment (start 142.038 106.485) (end 139.498 109.025) (width 0.5) (layer B.Cu) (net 8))
 (segment (start 147.188 106.485) (end 142.038 106.485) (width 0.5) (layer B.Cu) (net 8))
 (segment (start 136.998 106.525) (end 139.498 109.025) (width 0.5) (layer B.Cu) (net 8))
 (segment (start 131.498 106.525) (end 136.998 106.525) (width 0.5) (layer B.Cu) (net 8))
 (segment (start 137.498 101.945) (end 142.038 106.485) (width 0.5) (layer B.Cu) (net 8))
 (segment (start 137.498 86.365) (end 137.498 101.945) (width 0.5) (layer B.Cu) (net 8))
 (via (at 154.498 116.365) (size 1.8) (drill 0.8) (layers F.Cu B.Cu) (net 8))
 (segment (start 149.998 116.365) (end 154.498 116.365) (width 0.5) (layer F.Cu) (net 8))
 (segment (start 147.498 113.865) (end 149.998 116.365) (width 0.5) (layer F.Cu) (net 8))
 (segment (start 154.498 123.505) (end 154.178 123.825) (width 0.5) (layer B.Cu) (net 8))
 (segment (start 154.498 116.365) (end 154.498 123.505) (width 0.5) (layer B.Cu) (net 8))
 (segment (start 114.498 110.590997) (end 116.55567 112.648667) (width 0.5) (layer F.Cu) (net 8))
 (segment (start 114.498 103.365) (end 114.498 110.590997) (width 0.5) (layer F.Cu) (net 8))
 (segment (start 176.167998 113.145) (end 176.998 113.145) (width 0.5) (layer F.Cu) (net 8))
 (segment (start 172.947998 116.365) (end 176.167998 113.145) (width 0.5) (layer F.Cu) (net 8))
 (segment (start 154.498 116.365) (end 172.947998 116.365) (width 0.5) (layer F.Cu) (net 8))
 (segment (start 147.188 113.555) (end 147.498 113.865) (width 0.5) (layer B.Cu) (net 8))
 (segment (start 147.188 106.485) (end 147.188 113.555) (width 0.5) (layer B.Cu) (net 8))
 (segment (start 137.498 75.649) (end 137.414 75.565) (width 0.5) (layer F.Cu) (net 8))
 (segment (start 137.498 86.365) (end 137.498 75.649) (width 0.5) (layer F.Cu) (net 8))
 (segment (start 166.998 123.705) (end 166.878 123.825) (width 0.5) (layer B.Cu) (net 18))
 (via (at 124.998 118.365) (size 1.8) (drill 0.8) (layers F.Cu B.Cu) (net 18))
 (segment (start 124.870914 118.492086) (end 124.998 118.365) (width 0.5) (layer F.Cu) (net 18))
 (segment (start 116.968421 118.492086) (end 124.870914 118.492086) (width 0.5) (layer F.Cu) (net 18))
 (segment (start 115.205669 116.729334) (end 116.968421 118.492086) (width 0.5) (layer F.Cu) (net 18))
 (segment (start 115.205669 115.157331) (end 115.205669 116.729334) (width 0.5) (layer F.Cu) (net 18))
 (segment (start 115.998 114.365) (end 115.205669 115.157331) (width 0.5) (layer F.Cu) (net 18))
 (via (at 148.998 121.365) (size 1.8) (drill 0.8) (layers F.Cu B.Cu) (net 18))
 (segment (start 127.998 121.365) (end 148.998 121.365) (width 0.5) (layer B.Cu) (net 18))
 (segment (start 124.998 118.365) (end 127.998 121.365) (width 0.5) (layer B.Cu) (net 18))
 (segment (start 166.772389 123.825) (end 166.878 123.825) (width 0.5) (layer F.Cu) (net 18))
 (segment (start 164.312389 121.365) (end 166.772389 123.825) (width 0.5) (layer F.Cu) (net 18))
 (segment (start 148.998 121.365) (end 164.312389 121.365) (width 0.5) (layer F.Cu) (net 18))
 (via (at 163.498 118.865) (size 1.8) (drill 0.8) (layers F.Cu B.Cu) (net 6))
 (segment (start 174.298 108.065) (end 163.498 118.865) (width 0.5) (layer B.Cu) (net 6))
 (segment (start 176.998 108.065) (end 174.298 108.065) (width 0.5) (layer B.Cu) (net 6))
 (segment (start 146.558 121.102153) (end 146.558 123.825) (width 0.5) (layer F.Cu) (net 6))
 (segment (start 148.251183 119.40897) (end 146.558 121.102153) (width 0.5) (layer F.Cu) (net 6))
 (segment (start 162.954013 119.408986) (end 148.251183 119.40897) (width 0.5) (layer F.Cu) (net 6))
 (segment (start 163.498 118.865) (end 162.954013 119.408986) (width 0.5) (layer F.Cu) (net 6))
 (segment (start 126.498 111.865) (end 126.498 96.365) (width 0.5) (layer B.Cu) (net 12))
 (segment (start 131.498 96.365) (end 126.498 96.365) (width 0.5) (layer B.Cu) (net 12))
 (segment (start 142.148 96.365) (end 147.188 101.405) (width 0.5) (layer F.Cu) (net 12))
 (segment (start 131.498 96.365) (end 142.148 96.365) (width 0.5) (layer F.Cu) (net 12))
 (segment (start 170.498 98.525) (end 170.158 98.865) (width 0.5) (layer B.Cu) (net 9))
 (segment (start 156.768 103.365) (end 154.808 101.405) (width 0.5) (layer B.Cu) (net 9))
 (segment (start 161.498 103.365) (end 156.768 103.365) (width 0.5) (layer B.Cu) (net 9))
 (segment (start 165.658 103.365) (end 170.158 98.865) (width 0.5) (layer B.Cu) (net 9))
 (segment (start 161.498 103.365) (end 165.658 103.365) (width 0.5) (layer B.Cu) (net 9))
 (segment (start 166.658 95.365) (end 165.998 95.365) (width 0.5) (layer B.Cu) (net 9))
 (segment (start 170.158 98.865) (end 166.658 95.365) (width 0.5) (layer B.Cu) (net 9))
 (segment (start 144.498 96.175) (end 147.188 98.865) (width 0.5) (layer B.Cu) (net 10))
 (segment (start 160.323001 96.190001) (end 161.148002 95.365) (width 0.5) (layer B.Cu) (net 10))
 (segment (start 159.998 96.515002) (end 160.323001 96.190001) (width 0.5) (layer B.Cu) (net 10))
 (segment (start 159.998 98.865) (end 159.998 96.515002) (width 0.5) (layer B.Cu) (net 10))
 (segment (start 141.808 98.865) (end 144.498 96.175) (width 0.5) (layer B.Cu) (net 10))
 (segment (start 139.498 98.865) (end 141.808 98.865) (width 0.5) (layer B.Cu) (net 10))
 (segment (start 159.998 96.365) (end 160.998 95.365) (width 0.5) (layer B.Cu) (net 10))
 (segment (start 159.998 98.865) (end 159.998 96.365) (width 0.5) (layer B.Cu) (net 10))
 (via (at 144.498 87.865) (size 1.8) (drill 0.8) (layers F.Cu B.Cu) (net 10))
 (segment (start 160.998 94.23363) (end 154.62937 87.865) (width 0.5) (layer B.Cu) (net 10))
 (segment (start 154.62937 87.865) (end 144.498 87.865) (width 0.5) (layer B.Cu) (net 10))
 (segment (start 160.998 95.365) (end 160.998 94.23363) (width 0.5) (layer B.Cu) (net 10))
 (via (at 144.498 91.365) (size 1.8) (drill 0.8) (layers F.Cu B.Cu) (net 10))
 (segment (start 144.498 87.865) (end 144.498 91.365) (width 0.5) (layer F.Cu) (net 10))
 (segment (start 144.498 91.365) (end 144.498 96.175) (width 0.5) (layer B.Cu) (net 10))
 (segment (start 152.838 113.525) (end 152.498 113.865) (width 0.5) (layer B.Cu) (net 19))
 (segment (start 161.498 113.525) (end 152.838 113.525) (width 0.5) (layer B.Cu) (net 19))
 (segment (start 161.498 123.525) (end 161.798 123.825) (width 0.5) (layer B.Cu) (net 19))
 (segment (start 161.498 113.525) (end 161.498 123.525) (width 0.5) (layer B.Cu) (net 19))
 (segment (start 119.82033 117.990613) (end 119.82033 117.142085) (width 0.5) (layer B.Cu) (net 16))
 (segment (start 116.601655 118.492086) (end 119.318857 118.492086) (width 0.5) (layer B.Cu) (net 16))
 (segment (start 113.447979 115.33841) (end 116.601655 118.492086) (width 0.5) (layer B.Cu) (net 16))
 (segment (start 113.447979 112.344127) (end 113.447979 115.33841) (width 0.5) (layer B.Cu) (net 16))
 (segment (start 120.498 105.294106) (end 113.447979 112.344127) (width 0.5) (layer B.Cu) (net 16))
 (segment (start 120.498 75.865) (end 120.498 105.294106) (width 0.5) (layer B.Cu) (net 16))
 (segment (start 119.318857 118.492086) (end 119.82033 117.990613) (width 0.5) (layer B.Cu) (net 16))
 (via (at 116.498 106.365) (size 1.8) (drill 0.8) (layers F.Cu B.Cu) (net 13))
 (segment (start 118.01567 107.88267) (end 116.498 106.365) (width 0.5) (layer F.Cu) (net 13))
 (segment (start 118.01567 111.587915) (end 118.01567 107.88267) (width 0.5) (layer F.Cu) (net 13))
 (segment (start 116.498 106.365) (end 116.498 75.865) (width 0.5) (layer B.Cu) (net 13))
 (segment (start 114.44799 112.758345) (end 114.44799 114.924192) (width 0.5) (layer B.Cu) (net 17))
 (segment (start 114.44799 114.924192) (end 115.605131 116.081333) (width 0.5) (layer B.Cu) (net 17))
 (segment (start 121.498011 105.708324) (end 114.44799 112.758345) (width 0.5) (layer B.Cu) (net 17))
 (segment (start 115.605131 116.081333) (end 116.55567 116.081333) (width 0.5) (layer B.Cu) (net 17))
 (segment (start 121.498011 84.864989) (end 121.498011 105.708324) (width 0.5) (layer B.Cu) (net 17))
 (segment (start 124.498 81.865) (end 121.498011 84.864989) (width 0.5) (layer B.Cu) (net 17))
 (segment (start 126.498 81.865) (end 126.498 86.205) (width 0.5) (layer B.Cu) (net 20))
 (segment (start 122.498022 111.430975) (end 121.28033 112.648667) (width 0.5) (layer B.Cu) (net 15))
 (segment (start 122.498022 92.49898) (end 122.498022 111.430975) (width 0.5) (layer B.Cu) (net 15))
 (segment (start 128.498 81.865) (end 128.498 86.499002) (width 0.5) (layer B.Cu) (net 15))
 (segment (start 128.498 86.499002) (end 122.498022 92.49898) (width 0.5) (layer B.Cu) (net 15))
 (segment (start 119.82033 106.578328) (end 119.82033 111.587915) (width 0.5) (layer F.Cu) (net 14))
 (segment (start 114.607002 101.365) (end 119.82033 106.578328) (width 0.5) (layer F.Cu) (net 14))
 (segment (start 114.498 101.365) (end 114.607002 101.365) (width 0.5) (layer F.Cu) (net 14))
 (segment (start 152.29399 85.36499) (end 142.494 75.565) (width 0.5) (layer B.Cu) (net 5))
 (segment (start 171.708001 98.120999) (end 158.951992 85.36499) (width 0.5) (layer B.Cu) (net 5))
 (segment (start 171.708001 101.997001) (end 171.708001 98.120999) (width 0.5) (layer B.Cu) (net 5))
 (segment (start 175.236 105.525) (end 171.708001 101.997001) (width 0.5) (layer B.Cu) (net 5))
 (segment (start 176.998 105.525) (end 175.236 105.525) (width 0.5) (layer B.Cu) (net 5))
 (segment (start 158.951992 85.36499) (end 152.29399 85.36499) (width 0.5) (layer B.Cu) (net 5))
 (segment (start 176.998 97.905) (end 176.538 97.905) (width 0.5) (layer B.Cu) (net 2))
 (segment (start 159.366211 84.364979) (end 153.833979 84.364979) (width 0.5) (layer B.Cu) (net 2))
 (segment (start 153.833979 84.364979) (end 145.034 75.565) (width 0.5) (layer B.Cu) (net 2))
 (segment (start 176.998 97.905) (end 172.906232 97.905) (width 0.5) (layer B.Cu) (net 2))
 (segment (start 172.906232 97.905) (end 159.366211 84.364979) (width 0.5) (layer B.Cu) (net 2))
 (segment (start 149.34001 77.33101) (end 147.574 75.565) (width 0.5) (layer B.Cu) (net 1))
 (segment (start 153.74647 77.33101) (end 149.34001 77.33101) (width 0.5) (layer B.Cu) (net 1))
 (segment (start 171.78046 95.365) (end 153.74647 77.33101) (width 0.5) (layer B.Cu) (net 1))
 (segment (start 176.998 95.365) (end 171.78046 95.365) (width 0.5) (layer B.Cu) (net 1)))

